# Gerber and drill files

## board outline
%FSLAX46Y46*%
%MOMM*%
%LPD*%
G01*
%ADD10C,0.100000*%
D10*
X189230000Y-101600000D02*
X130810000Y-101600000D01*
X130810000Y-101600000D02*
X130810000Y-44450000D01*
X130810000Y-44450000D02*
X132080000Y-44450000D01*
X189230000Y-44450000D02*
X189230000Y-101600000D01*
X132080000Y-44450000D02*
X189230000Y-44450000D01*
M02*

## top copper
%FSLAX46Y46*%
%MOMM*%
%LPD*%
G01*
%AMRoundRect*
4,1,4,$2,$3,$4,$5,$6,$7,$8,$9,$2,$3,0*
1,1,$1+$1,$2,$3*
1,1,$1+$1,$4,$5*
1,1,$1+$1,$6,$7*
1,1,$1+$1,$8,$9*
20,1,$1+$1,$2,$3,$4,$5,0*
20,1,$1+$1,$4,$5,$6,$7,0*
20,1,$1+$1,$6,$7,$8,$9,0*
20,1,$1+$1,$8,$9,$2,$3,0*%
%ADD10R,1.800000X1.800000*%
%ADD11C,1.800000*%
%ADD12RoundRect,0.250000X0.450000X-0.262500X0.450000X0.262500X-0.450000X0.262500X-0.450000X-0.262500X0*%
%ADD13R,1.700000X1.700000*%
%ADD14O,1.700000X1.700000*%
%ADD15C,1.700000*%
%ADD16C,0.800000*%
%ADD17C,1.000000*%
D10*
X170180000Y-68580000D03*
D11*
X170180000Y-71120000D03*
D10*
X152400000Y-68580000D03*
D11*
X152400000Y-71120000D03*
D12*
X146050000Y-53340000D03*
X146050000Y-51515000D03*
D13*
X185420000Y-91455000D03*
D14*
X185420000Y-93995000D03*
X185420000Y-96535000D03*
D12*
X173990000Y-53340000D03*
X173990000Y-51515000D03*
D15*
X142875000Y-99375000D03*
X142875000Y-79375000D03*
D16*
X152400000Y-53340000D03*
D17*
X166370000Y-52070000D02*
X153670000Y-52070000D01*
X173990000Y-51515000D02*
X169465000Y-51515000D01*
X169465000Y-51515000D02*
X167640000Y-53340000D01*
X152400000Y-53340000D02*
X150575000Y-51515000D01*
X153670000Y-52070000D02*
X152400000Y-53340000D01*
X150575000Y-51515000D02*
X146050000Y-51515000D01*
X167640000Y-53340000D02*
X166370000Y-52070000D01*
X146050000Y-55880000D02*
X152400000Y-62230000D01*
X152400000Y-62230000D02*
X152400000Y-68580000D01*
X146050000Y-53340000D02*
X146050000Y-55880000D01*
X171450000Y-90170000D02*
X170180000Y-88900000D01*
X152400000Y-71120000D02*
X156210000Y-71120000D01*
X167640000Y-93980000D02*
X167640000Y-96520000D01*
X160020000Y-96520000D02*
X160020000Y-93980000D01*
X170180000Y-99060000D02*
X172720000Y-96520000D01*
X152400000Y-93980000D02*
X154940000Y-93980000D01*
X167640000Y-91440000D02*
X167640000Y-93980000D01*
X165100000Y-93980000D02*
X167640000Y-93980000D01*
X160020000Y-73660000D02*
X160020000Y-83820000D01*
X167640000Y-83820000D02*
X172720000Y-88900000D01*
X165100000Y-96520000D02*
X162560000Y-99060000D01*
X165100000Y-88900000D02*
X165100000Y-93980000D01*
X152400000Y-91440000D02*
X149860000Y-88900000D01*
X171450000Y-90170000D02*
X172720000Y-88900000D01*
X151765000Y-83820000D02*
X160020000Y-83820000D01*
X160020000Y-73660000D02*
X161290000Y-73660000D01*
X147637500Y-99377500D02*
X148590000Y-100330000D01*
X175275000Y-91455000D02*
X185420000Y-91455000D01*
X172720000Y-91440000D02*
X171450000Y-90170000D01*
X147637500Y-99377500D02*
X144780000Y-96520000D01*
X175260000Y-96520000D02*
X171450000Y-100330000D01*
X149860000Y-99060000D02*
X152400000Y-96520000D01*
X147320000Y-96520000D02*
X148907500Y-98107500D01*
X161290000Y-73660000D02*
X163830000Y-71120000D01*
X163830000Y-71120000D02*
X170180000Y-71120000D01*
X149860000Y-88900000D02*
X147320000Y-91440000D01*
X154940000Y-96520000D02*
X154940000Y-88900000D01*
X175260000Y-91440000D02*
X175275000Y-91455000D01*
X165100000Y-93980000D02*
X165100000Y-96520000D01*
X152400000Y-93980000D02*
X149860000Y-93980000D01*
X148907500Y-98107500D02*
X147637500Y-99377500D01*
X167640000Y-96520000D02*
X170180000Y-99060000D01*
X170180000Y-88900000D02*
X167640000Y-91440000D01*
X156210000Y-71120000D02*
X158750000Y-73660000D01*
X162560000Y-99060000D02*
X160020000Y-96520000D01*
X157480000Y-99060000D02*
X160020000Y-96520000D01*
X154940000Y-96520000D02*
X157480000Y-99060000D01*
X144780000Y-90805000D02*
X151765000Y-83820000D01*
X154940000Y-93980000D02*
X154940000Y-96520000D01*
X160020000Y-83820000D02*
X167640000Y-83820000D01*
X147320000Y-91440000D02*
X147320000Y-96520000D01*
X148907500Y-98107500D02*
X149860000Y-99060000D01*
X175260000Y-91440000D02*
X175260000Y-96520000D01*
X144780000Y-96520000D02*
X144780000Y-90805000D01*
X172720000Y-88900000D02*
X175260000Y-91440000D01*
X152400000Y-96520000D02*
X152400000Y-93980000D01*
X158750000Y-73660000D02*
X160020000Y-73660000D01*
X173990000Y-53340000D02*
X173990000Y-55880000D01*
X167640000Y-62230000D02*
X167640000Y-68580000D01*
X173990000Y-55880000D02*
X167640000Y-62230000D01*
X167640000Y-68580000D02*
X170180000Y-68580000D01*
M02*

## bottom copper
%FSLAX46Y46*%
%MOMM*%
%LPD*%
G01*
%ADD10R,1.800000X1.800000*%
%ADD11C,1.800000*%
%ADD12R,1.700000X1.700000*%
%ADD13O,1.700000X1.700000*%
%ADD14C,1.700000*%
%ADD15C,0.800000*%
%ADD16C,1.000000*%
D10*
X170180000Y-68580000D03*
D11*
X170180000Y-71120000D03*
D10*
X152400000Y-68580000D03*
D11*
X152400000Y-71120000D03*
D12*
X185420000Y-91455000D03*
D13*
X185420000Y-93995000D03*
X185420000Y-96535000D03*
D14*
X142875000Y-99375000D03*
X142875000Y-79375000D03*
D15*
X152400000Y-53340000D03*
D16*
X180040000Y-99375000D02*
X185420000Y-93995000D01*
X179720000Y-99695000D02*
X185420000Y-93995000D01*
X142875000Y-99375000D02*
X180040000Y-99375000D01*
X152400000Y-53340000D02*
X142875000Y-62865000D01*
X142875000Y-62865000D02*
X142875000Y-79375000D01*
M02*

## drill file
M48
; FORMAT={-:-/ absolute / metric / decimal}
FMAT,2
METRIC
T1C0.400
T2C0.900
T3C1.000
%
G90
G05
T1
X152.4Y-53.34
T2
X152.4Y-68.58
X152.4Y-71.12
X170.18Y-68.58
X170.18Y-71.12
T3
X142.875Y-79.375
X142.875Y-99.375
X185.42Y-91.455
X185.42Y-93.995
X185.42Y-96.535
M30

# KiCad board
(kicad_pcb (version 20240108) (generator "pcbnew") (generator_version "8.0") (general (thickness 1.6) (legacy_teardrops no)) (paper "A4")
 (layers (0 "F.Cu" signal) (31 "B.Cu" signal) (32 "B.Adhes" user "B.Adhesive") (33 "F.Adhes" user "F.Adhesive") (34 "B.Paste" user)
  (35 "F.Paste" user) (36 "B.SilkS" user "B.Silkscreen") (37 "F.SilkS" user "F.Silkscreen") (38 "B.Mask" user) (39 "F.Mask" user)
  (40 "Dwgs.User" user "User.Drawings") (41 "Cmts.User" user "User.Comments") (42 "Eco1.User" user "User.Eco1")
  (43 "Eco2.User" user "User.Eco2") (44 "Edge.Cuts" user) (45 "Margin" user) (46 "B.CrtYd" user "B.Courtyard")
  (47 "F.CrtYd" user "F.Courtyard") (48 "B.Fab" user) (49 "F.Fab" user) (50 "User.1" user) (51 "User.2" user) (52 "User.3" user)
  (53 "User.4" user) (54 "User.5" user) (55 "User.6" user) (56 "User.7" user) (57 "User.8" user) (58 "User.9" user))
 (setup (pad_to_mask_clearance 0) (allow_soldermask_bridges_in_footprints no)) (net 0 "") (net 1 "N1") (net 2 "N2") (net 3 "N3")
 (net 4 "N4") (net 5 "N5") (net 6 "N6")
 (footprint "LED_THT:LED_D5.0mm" (layer "F.Cu") (at 170.18 68.58 -90)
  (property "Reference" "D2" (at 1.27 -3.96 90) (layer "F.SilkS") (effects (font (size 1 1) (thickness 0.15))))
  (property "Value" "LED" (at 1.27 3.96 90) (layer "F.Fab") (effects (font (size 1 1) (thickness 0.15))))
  (pad "1" thru_hole rect (at 0 0 270) (size 1.8 1.8) (drill 0.9) (layers "*.Cu" "*.Mask") (remove_unused_layers no) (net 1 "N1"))
  (pad "2" thru_hole circle (at 2.54 0 270) (size 1.8 1.8) (drill 0.9) (layers "*.Cu" "*.Mask") (remove_unused_layers no) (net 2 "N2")))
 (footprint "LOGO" (layer "F.Cu") (at 160.02 66.04)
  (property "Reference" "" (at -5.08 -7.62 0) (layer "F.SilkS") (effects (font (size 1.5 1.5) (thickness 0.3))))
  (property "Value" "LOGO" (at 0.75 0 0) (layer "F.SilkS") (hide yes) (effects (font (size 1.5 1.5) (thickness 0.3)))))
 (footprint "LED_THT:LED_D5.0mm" (layer "F.Cu") (at 152.4 68.58 -90)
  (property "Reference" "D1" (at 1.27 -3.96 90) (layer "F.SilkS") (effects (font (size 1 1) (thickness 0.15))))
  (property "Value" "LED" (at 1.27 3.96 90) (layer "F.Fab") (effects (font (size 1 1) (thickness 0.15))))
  (pad "1" thru_hole rect (at 0 0 270) (size 1.8 1.8) (drill 0.9) (layers "*.Cu" "*.Mask") (remove_unused_layers no) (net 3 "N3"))
  (pad "2" thru_hole circle (at 2.54 0 270) (size 1.8 1.8) (drill 0.9) (layers "*.Cu" "*.Mask") (remove_unused_layers no) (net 2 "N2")))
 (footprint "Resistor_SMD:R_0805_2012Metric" (layer "F.Cu") (at 146.05 52.4275 90)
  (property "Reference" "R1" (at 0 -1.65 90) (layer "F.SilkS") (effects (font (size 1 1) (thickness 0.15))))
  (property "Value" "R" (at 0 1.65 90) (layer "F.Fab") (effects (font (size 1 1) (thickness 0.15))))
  (pad "1" smd roundrect (at -0.9125 0 90) (size 1.025 1.4) (layers "F.Cu" "F.Paste" "F.Mask") (roundrect_rratio 0.243902) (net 3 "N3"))
  (pad "2" smd roundrect (at 0.9125 0 90) (size 1.025 1.4) (layers "F.Cu" "F.Paste" "F.Mask") (roundrect_rratio 0.243902) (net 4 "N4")))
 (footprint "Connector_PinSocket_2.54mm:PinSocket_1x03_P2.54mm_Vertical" (layer "F.Cu") (at 185.42 91.455)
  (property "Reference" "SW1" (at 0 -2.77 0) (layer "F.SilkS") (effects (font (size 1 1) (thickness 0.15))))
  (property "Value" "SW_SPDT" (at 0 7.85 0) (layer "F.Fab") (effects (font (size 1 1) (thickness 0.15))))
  (pad "1" thru_hole rect (at 0 0) (size 1.7 1.7) (drill 1) (layers "*.Cu" "*.Mask") (remove_unused_layers no) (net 2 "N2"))
  (pad "2" thru_hole oval (at 0 2.54) (size 1.7 1.7) (drill 1) (layers "*.Cu" "*.Mask") (remove_unused_layers no) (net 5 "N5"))
  (pad "3" thru_hole oval (at 0 5.08) (size 1.7 1.7) (drill 1) (layers "*.Cu" "*.Mask") (remove_unused_layers no) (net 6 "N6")))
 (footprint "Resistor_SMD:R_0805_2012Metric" (layer "F.Cu") (at 173.99 52.4275 90)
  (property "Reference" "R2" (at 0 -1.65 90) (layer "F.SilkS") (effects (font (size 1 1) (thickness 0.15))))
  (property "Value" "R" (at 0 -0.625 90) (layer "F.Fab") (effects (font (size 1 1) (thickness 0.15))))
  (pad "1" smd roundrect (at -0.9125 0 90) (size 1.025 1.4) (layers "F.Cu" "F.Paste" "F.Mask") (roundrect_rratio 0.243902) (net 1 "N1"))
  (pad "2" smd roundrect (at 0.9125 0 90) (size 1.025 1.4) (layers "F.Cu" "F.Paste" "F.Mask") (roundrect_rratio 0.243902) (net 4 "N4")))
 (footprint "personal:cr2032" (layer "B.Cu") (at 142.875 99.375 90)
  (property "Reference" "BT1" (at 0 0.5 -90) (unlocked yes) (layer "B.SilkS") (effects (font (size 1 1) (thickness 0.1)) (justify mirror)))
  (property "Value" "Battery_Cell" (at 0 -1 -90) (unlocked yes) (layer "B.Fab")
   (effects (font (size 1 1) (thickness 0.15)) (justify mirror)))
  (pad "1" thru_hole circle (at 0 0 90) (size 1.7 1.7) (drill 1) (layers "*.Cu" "*.Mask") (remove_unused_layers no) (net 5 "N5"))
  (pad "2" thru_hole circle (at 20 0 90) (size 1.7 1.7) (drill 1) (layers "*.Cu" "*.Mask") (remove_unused_layers no) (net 4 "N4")))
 (gr_line (start 189.23 101.6) (end 130.81 101.6) (stroke (width 0.1) (type default)) (layer "Edge.Cuts"))
 (gr_line (start 130.81 101.6) (end 130.81 44.45) (stroke (width 0.1) (type default)) (layer "Edge.Cuts"))
 (gr_line (start 130.81 44.45) (end 132.08 44.45) (stroke (width 0.1) (type default)) (layer "Edge.Cuts"))
 (gr_line (start 189.23 44.45) (end 189.23 101.6) (stroke (width 0.1) (type default)) (layer "Edge.Cuts"))
 (gr_line (start 132.08 44.45) (end 189.23 44.45) (stroke (width 0.1) (type default)) (layer "Edge.Cuts"))
 (segment (start 180.04 99.375) (end 185.42 93.995) (width 1) (layer "B.Cu") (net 5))
 (segment (start 179.72 99.695) (end 185.42 93.995) (width 1) (layer "B.Cu") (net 5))
 (segment (start 142.875 99.375) (end 180.04 99.375) (width 1) (layer "B.Cu") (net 5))
 (segment (start 166.37 52.07) (end 153.67 52.07) (width 1) (layer "F.Cu") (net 4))
 (segment (start 173.99 51.515) (end 169.465 51.515) (width 1) (layer "F.Cu") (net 4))
 (segment (start 169.465 51.515) (end 167.64 53.34) (width 1) (layer "F.Cu") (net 4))
 (segment (start 152.4 53.34) (end 150.575 51.515) (width 1) (layer "F.Cu") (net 4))
 (segment (start 153.67 52.07) (end 152.4 53.34) (width 1) (layer "F.Cu") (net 4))
 (segment (start 150.575 51.515) (end 146.05 51.515) (width 1) (layer "F.Cu") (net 4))
 (segment (start 167.64 53.34) (end 166.37 52.07) (width 1) (layer "F.Cu") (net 4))
 (via (at 152.4 53.34) (size 0.8) (drill 0.4) (layers "F.Cu" "B.Cu") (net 4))
 (segment (start 152.4 53.34) (end 142.875 62.865) (width 1) (layer "B.Cu") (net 4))
 (segment (start 142.875 62.865) (end 142.875 79.375) (width 1) (layer "B.Cu") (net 4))
 (segment (start 146.05 55.88) (end 152.4 62.23) (width 1) (layer "F.Cu") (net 3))
 (segment (start 152.4 62.23) (end 152.4 68.58) (width 1) (layer "F.Cu") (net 3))
 (segment (start 146.05 53.34) (end 146.05 55.88) (width 1) (layer "F.Cu") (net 3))
 (segment (start 171.45 90.17) (end 170.18 88.9) (width 1) (layer "F.Cu") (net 2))
 (segment (start 152.4 71.12) (end 156.21 71.12) (width 1) (layer "F.Cu") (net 2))
 (segment (start 167.64 93.98) (end 167.64 96.52) (width 1) (layer "F.Cu") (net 2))
 (segment (start 160.02 96.52) (end 160.02 93.98) (width 1) (layer "F.Cu") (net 2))
 (segment (start 170.18 99.06) (end 172.72 96.52) (width 1) (layer "F.Cu") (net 2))
 (segment (start 152.4 93.98) (end 154.94 93.98) (width 1) (layer "F.Cu") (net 2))
 (segment (start 167.64 91.44) (end 167.64 93.98) (width 1) (layer "F.Cu") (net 2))
 (segment (start 165.1 93.98) (end 167.64 93.98) (width 1) (layer "F.Cu") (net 2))
 (segment (start 160.02 73.66) (end 160.02 83.82) (width 1) (layer "F.Cu") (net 2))
 (segment (start 167.64 83.82) (end 172.72 88.9) (width 1) (layer "F.Cu") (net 2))
 (segment (start 165.1 96.52) (end 162.56 99.06) (width 1) (layer "F.Cu") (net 2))
 (segment (start 165.1 88.9) (end 165.1 93.98) (width 1) (layer "F.Cu") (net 2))
 (segment (start 152.4 91.44) (end 149.86 88.9) (width 1) (layer "F.Cu") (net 2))
 (segment (start 171.45 90.17) (end 172.72 88.9) (width 1) (layer "F.Cu") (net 2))
 (segment (start 151.765 83.82) (end 160.02 83.82) (width 1) (layer "F.Cu") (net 2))
 (segment (start 160.02 73.66) (end 161.29 73.66) (width 1) (layer "F.Cu") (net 2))
 (segment (start 147.6375 99.3775) (end 148.59 100.33) (width 1) (layer "F.Cu") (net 2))
 (segment (start 175.275 91.455) (end 185.42 91.455) (width 1) (layer "F.Cu") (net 2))
 (segment (start 172.72 91.44) (end 171.45 90.17) (width 1) (layer "F.Cu") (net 2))
 (segment (start 147.6375 99.3775) (end 144.78 96.52) (width 1) (layer "F.Cu") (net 2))
 (segment (start 175.26 96.52) (end 171.45 100.33) (width 1) (layer "F.Cu") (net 2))
 (segment (start 149.86 99.06) (end 152.4 96.52) (width 1) (layer "F.Cu") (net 2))
 (segment (start 147.32 96.52) (end 148.9075 98.1075) (width 1) (layer "F.Cu") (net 2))
 (segment (start 161.29 73.66) (end 163.83 71.12) (width 1) (layer "F.Cu") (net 2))
 (segment (start 163.83 71.12) (end 170.18 71.12) (width 1) (layer "F.Cu") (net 2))
 (segment (start 149.86 88.9) (end 147.32 91.44) (width 1) (layer "F.Cu") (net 2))
 (segment (start 154.94 96.52) (end 154.94 88.9) (width 1) (layer "F.Cu") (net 2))
 (segment (start 175.26 91.44) (end 175.275 91.455) (width 1) (layer "F.Cu") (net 2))
 (segment (start 165.1 93.98) (end 165.1 96.52) (width 1) (layer "F.Cu") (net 2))
 (segment (start 152.4 93.98) (end 149.86 93.98) (width 1) (layer "F.Cu") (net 2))
 (segment (start 148.9075 98.1075) (end 147.6375 99.3775) (width 1) (layer "F.Cu") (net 2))
 (segment (start 167.64 96.52) (end 170.18 99.06) (width 1) (layer "F.Cu") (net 2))
 (segment (start 170.18 88.9) (end 167.64 91.44) (width 1) (layer "F.Cu") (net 2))
 (segment (start 156.21 71.12) (end 158.75 73.66) (width 1) (layer "F.Cu") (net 2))
 (segment (start 162.56 99.06) (end 160.02 96.52) (width 1) (layer "F.Cu") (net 2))
 (segment (start 157.48 99.06) (end 160.02 96.52) (width 1) (layer "F.Cu") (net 2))
 (segment (start 154.94 96.52) (end 157.48 99.06) (width 1) (layer "F.Cu") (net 2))
 (segment (start 144.78 90.805) (end 151.765 83.82) (width 1) (layer "F.Cu") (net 2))
 (segment (start 154.94 93.98) (end 154.94 96.52) (width 1) (layer "F.Cu") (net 2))
 (segment (start 160.02 83.82) (end 167.64 83.82) (width 1) (layer "F.Cu") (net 2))
 (segment (start 147.32 91.44) (end 147.32 96.52) (width 1) (layer "F.Cu") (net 2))
 (segment (start 148.9075 98.1075) (end 149.86 99.06) (width 1) (layer "F.Cu") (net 2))
 (segment (start 175.26 91.44) (end 175.26 96.52) (width 1) (layer "F.Cu") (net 2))
 (segment (start 144.78 96.52) (end 144.78 90.805) (width 1) (layer "F.Cu") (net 2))
 (segment (start 172.72 88.9) (end 175.26 91.44) (width 1) (layer "F.Cu") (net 2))
 (segment (start 152.4 96.52) (end 152.4 93.98) (width 1) (layer "F.Cu") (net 2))
 (segment (start 158.75 73.66) (end 160.02 73.66) (width 1) (layer "F.Cu") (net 2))
 (segment (start 173.99 53.34) (end 173.99 55.88) (width 1) (layer "F.Cu") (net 1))
 (segment (start 167.64 62.23) (end 167.64 68.58) (width 1) (layer "F.Cu") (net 1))
 (segment (start 173.99 55.88) (end 167.64 62.23) (width 1) (layer "F.Cu") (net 1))
 (segment (start 167.64 68.58) (end 170.18 68.58) (width 1) (layer "F.Cu") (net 1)))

